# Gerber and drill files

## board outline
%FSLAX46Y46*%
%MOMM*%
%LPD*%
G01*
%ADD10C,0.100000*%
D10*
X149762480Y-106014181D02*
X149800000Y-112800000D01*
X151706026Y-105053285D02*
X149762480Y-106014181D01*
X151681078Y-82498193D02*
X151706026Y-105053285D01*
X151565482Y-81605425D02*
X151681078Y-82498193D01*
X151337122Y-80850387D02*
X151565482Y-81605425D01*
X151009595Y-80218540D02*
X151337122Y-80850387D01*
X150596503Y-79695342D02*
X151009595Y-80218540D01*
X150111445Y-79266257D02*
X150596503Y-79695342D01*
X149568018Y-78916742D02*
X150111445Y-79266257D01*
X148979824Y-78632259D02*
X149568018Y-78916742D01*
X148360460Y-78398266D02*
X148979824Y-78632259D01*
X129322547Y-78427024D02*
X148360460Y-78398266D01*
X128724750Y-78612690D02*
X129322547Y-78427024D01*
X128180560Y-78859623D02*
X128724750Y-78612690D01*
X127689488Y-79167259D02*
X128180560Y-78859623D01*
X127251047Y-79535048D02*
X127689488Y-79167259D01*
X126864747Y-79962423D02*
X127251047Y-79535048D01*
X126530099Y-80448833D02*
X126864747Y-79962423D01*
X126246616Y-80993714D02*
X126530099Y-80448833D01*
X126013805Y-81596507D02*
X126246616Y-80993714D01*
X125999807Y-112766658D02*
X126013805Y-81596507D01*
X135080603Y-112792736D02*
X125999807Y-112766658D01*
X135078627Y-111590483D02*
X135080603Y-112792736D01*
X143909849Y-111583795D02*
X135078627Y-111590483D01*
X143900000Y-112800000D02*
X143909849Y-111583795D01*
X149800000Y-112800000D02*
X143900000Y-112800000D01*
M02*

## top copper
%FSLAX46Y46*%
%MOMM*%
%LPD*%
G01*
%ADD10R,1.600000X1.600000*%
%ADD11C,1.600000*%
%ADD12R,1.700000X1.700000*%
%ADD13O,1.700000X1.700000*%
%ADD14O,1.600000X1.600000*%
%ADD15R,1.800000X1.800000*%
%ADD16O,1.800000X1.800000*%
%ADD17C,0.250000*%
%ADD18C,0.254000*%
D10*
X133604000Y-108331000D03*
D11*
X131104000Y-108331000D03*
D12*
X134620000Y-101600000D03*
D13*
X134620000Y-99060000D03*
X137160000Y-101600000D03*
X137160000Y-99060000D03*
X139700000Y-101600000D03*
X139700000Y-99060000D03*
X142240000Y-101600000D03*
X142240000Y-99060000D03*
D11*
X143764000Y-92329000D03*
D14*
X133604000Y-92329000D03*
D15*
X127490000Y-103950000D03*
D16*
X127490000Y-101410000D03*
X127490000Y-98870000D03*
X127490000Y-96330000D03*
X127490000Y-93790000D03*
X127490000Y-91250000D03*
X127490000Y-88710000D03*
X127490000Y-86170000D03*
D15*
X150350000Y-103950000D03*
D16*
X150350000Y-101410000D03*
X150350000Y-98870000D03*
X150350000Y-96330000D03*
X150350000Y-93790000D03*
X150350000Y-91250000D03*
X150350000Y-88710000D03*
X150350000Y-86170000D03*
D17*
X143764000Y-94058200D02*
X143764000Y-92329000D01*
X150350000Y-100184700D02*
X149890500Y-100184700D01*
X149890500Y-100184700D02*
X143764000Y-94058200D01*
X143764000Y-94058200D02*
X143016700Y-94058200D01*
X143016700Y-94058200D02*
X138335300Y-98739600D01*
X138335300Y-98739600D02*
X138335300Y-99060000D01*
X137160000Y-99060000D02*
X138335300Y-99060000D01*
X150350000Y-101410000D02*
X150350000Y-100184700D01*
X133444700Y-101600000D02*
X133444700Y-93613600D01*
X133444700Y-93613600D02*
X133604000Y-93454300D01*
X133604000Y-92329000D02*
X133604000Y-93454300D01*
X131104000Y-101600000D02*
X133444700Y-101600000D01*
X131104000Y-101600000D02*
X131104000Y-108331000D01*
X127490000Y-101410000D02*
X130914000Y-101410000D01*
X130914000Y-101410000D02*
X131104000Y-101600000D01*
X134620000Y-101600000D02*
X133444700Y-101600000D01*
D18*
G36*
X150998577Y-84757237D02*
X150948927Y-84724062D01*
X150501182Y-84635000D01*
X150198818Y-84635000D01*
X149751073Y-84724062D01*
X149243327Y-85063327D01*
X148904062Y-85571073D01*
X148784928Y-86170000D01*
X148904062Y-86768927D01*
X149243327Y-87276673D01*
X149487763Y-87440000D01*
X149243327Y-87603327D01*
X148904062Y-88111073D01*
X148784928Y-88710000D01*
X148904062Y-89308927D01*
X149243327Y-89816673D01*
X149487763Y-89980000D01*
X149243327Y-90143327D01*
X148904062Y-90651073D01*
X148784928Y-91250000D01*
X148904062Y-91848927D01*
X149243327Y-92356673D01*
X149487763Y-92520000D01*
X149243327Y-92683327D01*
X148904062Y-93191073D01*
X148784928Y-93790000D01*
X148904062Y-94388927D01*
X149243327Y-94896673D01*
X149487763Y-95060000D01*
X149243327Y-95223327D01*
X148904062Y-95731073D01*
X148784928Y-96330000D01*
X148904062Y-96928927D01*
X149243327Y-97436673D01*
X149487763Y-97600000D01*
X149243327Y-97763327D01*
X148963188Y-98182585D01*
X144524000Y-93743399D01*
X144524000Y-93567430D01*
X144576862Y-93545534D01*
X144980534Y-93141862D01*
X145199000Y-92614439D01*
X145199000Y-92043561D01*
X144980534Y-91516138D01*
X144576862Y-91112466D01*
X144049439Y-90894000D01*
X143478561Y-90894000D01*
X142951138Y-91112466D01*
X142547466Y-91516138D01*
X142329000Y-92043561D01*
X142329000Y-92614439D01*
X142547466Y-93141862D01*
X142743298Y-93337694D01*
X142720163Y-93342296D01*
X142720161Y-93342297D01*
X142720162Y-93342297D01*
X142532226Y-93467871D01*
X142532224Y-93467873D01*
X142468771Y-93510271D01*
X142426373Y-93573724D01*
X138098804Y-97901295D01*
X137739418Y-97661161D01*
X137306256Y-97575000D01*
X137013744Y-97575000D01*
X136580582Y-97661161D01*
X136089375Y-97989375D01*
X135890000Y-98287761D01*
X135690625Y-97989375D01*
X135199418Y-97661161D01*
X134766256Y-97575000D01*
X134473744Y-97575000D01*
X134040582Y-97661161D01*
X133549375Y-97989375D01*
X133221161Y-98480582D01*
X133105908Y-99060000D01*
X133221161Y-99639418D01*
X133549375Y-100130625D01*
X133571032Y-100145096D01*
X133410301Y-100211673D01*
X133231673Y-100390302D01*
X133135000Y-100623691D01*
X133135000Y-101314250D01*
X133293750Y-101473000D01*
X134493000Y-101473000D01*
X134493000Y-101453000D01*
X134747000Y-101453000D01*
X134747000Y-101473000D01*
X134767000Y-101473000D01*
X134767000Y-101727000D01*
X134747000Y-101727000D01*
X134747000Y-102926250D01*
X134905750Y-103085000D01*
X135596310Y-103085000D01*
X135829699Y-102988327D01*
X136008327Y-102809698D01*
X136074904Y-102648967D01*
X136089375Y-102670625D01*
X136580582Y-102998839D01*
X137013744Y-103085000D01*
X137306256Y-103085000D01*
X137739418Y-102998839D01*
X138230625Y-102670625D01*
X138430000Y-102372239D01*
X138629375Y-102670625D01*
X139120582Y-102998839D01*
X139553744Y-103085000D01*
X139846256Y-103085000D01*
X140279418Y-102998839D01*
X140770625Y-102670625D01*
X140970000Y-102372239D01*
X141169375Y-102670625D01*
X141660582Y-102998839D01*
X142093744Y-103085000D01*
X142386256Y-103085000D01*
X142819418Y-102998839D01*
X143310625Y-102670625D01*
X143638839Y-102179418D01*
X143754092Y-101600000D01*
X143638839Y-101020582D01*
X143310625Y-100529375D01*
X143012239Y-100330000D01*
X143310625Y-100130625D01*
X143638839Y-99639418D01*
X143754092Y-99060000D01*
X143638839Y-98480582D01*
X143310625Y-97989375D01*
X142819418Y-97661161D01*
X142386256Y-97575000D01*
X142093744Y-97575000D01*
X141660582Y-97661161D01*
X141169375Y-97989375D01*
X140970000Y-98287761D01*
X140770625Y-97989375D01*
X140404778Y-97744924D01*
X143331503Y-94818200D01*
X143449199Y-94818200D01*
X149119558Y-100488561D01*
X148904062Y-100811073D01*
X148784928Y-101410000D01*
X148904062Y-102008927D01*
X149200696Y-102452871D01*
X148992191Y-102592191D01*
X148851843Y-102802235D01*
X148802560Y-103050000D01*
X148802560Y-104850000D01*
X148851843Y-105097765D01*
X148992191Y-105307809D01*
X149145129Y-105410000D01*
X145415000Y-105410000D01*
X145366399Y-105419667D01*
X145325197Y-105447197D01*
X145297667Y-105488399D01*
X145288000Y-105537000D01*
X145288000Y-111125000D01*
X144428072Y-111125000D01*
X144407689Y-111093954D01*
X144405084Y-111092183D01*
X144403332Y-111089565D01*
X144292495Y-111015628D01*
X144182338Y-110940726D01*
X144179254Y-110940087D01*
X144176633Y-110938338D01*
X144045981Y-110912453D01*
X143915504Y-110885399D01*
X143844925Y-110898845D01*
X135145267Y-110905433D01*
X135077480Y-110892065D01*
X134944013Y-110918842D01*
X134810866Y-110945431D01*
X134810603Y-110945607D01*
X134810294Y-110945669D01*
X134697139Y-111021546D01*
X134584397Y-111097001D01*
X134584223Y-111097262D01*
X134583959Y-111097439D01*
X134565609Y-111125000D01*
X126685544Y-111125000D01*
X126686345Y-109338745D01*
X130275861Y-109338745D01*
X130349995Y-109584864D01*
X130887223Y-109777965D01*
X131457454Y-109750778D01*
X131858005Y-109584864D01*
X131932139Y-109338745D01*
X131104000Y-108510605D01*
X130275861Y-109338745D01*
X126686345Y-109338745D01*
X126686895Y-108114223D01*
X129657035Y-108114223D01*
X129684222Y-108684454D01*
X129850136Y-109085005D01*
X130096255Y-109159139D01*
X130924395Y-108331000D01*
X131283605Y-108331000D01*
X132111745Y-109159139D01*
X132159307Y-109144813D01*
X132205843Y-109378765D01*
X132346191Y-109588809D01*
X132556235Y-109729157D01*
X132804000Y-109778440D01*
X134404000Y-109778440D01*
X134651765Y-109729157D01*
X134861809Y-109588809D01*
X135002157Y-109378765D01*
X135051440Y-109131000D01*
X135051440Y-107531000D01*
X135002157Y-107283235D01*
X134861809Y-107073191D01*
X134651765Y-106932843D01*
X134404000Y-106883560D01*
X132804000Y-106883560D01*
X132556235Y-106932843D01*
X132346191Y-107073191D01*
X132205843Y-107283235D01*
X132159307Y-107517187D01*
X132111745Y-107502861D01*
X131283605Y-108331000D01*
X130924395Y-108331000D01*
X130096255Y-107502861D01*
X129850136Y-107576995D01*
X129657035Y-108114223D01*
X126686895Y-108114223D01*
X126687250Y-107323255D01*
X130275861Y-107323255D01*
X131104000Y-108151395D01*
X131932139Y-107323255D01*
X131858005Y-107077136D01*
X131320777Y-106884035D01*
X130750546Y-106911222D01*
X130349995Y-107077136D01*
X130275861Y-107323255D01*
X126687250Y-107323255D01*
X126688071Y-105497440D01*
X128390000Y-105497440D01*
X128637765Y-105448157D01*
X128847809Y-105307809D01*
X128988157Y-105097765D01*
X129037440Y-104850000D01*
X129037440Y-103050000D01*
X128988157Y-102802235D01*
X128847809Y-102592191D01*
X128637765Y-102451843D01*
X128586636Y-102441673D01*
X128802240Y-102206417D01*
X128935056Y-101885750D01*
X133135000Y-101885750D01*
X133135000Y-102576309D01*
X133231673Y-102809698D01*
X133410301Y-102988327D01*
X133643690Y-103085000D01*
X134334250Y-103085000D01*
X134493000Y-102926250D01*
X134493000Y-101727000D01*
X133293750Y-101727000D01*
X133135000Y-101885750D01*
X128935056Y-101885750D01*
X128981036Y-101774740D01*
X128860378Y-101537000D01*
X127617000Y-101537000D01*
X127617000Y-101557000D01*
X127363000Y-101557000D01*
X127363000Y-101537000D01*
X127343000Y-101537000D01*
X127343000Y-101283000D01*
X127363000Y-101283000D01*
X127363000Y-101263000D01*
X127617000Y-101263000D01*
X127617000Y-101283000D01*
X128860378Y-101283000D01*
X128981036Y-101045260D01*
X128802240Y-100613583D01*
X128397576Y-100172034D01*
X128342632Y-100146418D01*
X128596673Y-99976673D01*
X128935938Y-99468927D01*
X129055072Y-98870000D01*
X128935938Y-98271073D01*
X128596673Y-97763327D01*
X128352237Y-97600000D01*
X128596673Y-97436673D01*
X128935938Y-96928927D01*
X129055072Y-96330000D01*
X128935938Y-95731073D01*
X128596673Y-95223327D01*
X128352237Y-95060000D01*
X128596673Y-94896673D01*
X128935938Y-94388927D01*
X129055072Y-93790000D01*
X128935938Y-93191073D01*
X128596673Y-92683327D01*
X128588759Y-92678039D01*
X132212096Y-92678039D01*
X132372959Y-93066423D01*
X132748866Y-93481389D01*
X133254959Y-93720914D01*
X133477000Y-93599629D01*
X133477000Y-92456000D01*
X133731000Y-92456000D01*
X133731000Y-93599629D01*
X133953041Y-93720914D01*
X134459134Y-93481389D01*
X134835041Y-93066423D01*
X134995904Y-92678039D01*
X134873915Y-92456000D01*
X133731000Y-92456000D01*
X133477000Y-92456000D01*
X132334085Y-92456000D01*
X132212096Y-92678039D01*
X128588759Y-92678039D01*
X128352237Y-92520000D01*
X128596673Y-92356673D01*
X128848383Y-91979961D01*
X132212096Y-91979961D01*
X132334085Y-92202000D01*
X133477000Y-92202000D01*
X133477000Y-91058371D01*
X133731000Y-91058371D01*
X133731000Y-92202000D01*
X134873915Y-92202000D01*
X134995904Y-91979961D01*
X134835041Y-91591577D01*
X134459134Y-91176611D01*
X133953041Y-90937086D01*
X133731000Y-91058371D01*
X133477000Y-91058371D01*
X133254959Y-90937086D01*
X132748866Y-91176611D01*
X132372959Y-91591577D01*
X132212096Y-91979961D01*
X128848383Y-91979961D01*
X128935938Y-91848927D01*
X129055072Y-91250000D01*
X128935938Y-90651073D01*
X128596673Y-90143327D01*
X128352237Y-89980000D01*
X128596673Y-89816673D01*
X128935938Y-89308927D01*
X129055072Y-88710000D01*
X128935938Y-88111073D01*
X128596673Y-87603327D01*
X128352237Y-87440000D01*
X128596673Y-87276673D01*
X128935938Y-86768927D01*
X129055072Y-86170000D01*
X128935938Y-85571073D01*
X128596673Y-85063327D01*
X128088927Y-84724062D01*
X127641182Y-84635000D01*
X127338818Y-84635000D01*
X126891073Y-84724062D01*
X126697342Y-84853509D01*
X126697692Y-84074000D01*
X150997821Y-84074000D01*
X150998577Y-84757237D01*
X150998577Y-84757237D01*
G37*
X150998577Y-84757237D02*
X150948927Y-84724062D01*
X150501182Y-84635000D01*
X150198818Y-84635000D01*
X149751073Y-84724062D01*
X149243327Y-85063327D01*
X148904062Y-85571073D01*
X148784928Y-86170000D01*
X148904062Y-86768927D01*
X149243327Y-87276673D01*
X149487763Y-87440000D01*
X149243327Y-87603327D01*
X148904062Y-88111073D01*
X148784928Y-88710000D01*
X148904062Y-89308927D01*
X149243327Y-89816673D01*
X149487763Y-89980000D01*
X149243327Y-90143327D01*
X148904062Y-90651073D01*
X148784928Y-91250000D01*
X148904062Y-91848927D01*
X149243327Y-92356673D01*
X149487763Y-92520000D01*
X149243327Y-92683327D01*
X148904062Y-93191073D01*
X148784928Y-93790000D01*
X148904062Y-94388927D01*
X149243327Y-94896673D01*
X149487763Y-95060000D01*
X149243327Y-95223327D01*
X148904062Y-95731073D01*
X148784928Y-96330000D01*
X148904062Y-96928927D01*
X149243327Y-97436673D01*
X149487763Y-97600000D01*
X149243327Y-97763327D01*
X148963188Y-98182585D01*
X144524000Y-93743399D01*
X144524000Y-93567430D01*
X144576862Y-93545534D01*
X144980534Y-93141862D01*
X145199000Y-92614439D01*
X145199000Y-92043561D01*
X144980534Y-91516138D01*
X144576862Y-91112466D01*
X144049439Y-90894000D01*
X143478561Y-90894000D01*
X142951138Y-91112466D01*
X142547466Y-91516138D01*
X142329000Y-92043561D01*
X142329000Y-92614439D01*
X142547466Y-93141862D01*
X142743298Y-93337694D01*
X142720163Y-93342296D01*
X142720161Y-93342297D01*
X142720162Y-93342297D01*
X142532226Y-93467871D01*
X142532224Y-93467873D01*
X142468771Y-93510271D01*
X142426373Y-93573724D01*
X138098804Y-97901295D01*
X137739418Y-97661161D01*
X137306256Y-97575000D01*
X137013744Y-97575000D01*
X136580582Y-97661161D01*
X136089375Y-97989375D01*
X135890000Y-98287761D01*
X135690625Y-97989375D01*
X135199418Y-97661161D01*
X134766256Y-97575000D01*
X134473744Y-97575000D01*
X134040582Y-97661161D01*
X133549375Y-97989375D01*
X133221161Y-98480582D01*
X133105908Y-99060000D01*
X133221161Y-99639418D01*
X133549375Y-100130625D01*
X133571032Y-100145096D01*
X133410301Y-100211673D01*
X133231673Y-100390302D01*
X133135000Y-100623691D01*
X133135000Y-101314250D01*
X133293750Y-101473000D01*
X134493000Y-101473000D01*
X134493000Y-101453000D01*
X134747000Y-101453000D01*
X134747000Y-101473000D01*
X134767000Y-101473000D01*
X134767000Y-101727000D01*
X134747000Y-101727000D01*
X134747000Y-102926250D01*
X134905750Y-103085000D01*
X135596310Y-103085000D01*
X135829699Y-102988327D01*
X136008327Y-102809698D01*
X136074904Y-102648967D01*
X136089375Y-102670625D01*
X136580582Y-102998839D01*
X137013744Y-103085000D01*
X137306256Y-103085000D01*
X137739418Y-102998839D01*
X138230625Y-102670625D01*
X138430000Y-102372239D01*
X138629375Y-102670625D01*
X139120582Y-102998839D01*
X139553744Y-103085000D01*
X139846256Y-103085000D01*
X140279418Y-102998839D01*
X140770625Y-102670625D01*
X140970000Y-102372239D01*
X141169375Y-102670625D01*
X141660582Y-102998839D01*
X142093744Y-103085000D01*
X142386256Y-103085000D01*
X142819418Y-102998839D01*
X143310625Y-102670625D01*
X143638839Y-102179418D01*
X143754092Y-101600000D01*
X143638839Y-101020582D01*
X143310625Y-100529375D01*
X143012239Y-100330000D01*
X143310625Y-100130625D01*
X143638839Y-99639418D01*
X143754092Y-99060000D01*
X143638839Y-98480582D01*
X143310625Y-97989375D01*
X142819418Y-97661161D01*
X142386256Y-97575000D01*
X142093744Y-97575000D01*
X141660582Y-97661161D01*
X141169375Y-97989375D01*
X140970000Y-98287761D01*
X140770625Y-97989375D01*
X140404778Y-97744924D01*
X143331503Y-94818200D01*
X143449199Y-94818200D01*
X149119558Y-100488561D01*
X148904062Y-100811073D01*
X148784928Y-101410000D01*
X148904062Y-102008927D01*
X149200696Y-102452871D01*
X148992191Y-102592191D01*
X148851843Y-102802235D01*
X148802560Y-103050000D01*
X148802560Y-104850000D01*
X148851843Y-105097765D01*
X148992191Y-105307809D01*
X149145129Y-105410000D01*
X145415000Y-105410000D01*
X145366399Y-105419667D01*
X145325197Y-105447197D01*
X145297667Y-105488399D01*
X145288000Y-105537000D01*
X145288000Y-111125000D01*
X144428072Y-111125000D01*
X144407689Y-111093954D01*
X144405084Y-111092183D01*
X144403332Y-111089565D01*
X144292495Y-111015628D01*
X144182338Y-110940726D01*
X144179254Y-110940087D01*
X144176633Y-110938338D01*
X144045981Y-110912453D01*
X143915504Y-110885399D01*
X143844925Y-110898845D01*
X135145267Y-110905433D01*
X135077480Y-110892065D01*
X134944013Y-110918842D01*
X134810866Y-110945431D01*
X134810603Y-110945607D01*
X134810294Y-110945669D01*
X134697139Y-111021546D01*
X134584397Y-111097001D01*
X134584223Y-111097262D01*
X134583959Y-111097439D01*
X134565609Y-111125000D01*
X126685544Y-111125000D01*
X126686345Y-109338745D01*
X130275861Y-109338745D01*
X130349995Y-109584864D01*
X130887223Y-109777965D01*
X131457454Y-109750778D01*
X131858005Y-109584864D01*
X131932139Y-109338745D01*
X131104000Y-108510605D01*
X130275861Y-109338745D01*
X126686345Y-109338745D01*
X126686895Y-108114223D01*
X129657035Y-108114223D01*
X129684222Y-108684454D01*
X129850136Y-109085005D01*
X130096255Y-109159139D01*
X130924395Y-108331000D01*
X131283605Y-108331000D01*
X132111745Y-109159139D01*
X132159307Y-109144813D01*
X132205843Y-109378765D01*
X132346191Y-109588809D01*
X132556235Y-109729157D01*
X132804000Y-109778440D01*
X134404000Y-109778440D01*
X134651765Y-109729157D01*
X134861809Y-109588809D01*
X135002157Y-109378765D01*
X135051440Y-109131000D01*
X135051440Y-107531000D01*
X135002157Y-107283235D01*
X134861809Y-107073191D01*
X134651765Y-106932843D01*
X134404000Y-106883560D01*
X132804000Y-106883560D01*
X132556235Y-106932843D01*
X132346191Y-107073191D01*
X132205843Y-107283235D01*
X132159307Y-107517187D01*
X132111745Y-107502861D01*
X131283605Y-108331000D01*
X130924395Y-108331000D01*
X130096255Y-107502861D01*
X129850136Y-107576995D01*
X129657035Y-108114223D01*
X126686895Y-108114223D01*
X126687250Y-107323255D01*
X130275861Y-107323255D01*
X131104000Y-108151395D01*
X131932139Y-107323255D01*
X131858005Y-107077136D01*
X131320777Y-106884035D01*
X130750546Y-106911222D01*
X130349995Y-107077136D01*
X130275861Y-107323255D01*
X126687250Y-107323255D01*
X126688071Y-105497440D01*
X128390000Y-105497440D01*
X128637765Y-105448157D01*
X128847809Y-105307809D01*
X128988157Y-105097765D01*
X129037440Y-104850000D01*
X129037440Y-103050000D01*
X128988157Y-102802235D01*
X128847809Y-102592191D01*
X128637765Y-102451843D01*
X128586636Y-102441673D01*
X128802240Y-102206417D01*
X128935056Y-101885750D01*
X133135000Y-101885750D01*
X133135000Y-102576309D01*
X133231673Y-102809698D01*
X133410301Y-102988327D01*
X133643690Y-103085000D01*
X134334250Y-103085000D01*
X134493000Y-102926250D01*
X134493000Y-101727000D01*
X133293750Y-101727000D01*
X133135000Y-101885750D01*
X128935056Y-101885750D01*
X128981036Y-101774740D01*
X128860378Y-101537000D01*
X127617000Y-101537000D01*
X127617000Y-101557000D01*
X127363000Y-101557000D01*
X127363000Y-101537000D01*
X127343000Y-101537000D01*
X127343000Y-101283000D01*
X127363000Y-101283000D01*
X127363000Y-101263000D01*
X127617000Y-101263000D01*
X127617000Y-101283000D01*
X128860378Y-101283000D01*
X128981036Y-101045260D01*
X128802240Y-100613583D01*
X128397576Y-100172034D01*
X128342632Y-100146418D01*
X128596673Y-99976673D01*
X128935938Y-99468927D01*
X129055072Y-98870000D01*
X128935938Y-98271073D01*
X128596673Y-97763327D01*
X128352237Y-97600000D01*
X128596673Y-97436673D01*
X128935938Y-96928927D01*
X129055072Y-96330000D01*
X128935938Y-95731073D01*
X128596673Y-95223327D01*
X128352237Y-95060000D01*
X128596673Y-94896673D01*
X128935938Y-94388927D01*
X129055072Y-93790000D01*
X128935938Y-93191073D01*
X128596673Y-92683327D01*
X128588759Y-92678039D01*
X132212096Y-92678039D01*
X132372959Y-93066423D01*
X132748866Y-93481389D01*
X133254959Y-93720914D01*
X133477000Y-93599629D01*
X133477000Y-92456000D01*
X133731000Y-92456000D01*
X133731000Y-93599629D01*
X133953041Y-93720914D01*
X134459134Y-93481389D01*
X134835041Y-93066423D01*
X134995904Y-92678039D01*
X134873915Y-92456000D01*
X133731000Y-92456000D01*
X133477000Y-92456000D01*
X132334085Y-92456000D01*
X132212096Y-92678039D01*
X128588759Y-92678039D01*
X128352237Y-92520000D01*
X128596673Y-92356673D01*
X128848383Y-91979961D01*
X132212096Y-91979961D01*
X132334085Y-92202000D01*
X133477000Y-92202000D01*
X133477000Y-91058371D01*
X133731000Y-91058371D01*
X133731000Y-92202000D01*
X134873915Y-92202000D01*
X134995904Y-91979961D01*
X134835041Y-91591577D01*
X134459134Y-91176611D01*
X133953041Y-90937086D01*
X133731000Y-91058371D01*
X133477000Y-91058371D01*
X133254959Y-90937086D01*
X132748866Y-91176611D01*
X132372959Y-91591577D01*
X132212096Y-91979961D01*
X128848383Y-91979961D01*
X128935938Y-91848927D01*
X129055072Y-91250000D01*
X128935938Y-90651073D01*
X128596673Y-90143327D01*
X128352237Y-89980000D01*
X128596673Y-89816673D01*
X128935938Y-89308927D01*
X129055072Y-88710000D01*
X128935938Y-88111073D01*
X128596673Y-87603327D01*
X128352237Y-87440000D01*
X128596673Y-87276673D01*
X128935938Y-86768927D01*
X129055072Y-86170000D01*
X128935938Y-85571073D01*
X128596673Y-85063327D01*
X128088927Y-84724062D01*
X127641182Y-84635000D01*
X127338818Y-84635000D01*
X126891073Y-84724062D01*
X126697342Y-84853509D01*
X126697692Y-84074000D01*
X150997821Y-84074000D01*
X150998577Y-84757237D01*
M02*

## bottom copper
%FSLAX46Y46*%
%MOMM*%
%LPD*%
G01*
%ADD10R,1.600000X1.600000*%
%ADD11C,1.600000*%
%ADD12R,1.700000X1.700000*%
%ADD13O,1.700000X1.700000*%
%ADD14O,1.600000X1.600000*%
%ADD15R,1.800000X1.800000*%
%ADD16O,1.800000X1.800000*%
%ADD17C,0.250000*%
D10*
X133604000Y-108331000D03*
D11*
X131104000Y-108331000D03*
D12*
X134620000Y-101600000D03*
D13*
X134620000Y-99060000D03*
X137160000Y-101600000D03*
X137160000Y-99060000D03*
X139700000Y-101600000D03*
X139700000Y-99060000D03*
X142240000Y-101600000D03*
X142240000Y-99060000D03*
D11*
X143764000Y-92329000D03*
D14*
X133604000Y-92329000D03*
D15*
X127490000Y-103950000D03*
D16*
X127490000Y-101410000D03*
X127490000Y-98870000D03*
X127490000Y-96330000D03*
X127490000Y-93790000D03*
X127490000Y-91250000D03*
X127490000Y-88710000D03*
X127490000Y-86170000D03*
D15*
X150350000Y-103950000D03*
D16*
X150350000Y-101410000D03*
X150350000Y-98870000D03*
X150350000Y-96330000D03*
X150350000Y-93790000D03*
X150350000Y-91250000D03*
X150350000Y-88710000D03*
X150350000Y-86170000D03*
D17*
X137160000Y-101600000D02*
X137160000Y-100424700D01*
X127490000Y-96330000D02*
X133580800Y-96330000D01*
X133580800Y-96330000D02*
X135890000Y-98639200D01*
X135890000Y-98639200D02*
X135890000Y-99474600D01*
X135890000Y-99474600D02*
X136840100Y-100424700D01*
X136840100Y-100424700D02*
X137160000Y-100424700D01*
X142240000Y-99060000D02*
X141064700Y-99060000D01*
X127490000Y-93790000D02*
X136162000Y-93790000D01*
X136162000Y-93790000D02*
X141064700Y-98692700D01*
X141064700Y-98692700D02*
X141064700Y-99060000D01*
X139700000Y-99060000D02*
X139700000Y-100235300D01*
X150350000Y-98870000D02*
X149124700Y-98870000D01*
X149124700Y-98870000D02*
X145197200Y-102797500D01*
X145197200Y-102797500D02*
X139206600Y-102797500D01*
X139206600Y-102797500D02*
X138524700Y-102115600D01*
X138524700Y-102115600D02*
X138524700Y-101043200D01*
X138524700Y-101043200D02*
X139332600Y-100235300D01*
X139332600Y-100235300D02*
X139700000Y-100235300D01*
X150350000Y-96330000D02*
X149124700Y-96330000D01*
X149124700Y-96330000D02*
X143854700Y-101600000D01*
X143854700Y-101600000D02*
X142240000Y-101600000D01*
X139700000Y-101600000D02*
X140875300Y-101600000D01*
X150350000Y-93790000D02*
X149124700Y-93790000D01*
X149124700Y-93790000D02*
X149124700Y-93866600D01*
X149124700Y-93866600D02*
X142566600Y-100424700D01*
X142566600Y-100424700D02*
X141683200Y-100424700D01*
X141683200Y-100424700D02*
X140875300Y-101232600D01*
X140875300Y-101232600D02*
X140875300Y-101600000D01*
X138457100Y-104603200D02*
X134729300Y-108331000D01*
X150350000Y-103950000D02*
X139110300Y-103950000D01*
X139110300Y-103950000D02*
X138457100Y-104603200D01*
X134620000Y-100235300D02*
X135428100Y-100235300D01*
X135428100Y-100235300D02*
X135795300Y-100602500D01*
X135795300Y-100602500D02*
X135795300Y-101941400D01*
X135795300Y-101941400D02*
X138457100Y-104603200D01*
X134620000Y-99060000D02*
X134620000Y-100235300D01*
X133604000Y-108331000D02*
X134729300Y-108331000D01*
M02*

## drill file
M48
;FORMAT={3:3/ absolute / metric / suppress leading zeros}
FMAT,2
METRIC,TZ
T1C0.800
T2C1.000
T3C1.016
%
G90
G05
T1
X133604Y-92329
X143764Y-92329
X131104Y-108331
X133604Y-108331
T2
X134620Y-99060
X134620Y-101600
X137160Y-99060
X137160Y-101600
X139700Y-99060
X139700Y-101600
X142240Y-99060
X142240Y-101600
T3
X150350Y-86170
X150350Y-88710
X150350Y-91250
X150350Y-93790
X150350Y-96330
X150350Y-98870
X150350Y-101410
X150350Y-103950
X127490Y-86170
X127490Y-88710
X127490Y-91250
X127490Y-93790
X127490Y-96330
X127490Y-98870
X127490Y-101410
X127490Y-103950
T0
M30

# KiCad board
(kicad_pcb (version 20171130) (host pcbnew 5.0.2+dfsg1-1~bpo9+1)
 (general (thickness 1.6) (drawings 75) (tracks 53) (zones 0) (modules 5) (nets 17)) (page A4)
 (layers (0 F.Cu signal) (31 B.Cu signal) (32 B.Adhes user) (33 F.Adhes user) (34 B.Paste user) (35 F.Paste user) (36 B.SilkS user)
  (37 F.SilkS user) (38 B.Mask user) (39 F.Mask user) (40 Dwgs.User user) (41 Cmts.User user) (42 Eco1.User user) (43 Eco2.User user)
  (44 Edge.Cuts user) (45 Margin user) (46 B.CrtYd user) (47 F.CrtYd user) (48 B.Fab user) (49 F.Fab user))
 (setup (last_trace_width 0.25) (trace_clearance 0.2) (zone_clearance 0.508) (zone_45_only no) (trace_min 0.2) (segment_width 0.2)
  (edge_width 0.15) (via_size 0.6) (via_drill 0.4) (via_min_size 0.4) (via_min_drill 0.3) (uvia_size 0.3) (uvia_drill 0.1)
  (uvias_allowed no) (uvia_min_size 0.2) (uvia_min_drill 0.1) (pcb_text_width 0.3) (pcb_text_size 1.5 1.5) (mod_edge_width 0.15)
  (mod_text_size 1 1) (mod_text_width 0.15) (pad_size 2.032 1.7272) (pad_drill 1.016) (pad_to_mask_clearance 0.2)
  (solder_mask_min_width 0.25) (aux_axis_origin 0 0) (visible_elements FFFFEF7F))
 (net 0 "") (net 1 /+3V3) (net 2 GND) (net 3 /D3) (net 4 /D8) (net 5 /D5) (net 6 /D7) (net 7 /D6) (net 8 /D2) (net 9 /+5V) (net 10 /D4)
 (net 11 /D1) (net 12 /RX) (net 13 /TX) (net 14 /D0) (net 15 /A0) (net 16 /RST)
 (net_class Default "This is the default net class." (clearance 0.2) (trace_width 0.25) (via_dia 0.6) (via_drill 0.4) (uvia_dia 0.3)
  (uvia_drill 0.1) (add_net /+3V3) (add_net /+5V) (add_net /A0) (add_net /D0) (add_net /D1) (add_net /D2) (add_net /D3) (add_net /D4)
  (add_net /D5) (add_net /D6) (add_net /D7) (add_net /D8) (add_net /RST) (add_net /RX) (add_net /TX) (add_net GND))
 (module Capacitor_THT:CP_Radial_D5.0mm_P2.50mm (layer F.Cu) (at 133.604 108.331 180)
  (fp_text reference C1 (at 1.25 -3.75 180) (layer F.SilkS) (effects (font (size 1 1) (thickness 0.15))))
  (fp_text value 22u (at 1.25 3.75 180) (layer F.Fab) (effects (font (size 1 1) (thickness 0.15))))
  (pad 1 thru_hole rect (at 0 0 180) (size 1.6 1.6) (drill 0.8) (layers *.Cu *.Mask) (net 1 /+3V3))
  (pad 2 thru_hole circle (at 2.5 0 180) (size 1.6 1.6) (drill 0.8) (layers *.Cu *.Mask) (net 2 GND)))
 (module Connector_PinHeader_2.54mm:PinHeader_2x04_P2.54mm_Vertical (layer F.Cu) (at 134.62 101.6 90)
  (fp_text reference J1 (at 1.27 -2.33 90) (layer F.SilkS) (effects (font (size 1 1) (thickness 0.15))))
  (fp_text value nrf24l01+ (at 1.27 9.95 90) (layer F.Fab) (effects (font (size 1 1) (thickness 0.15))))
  (pad 1 thru_hole rect (at 0 0 90) (size 1.7 1.7) (drill 1) (layers *.Cu *.Mask) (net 2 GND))
  (pad 2 thru_hole oval (at 2.54 0 90) (size 1.7 1.7) (drill 1) (layers *.Cu *.Mask) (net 1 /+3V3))
  (pad 3 thru_hole oval (at 0 2.54 90) (size 1.7 1.7) (drill 1) (layers *.Cu *.Mask) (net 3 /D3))
  (pad 4 thru_hole oval (at 2.54 2.54 90) (size 1.7 1.7) (drill 1) (layers *.Cu *.Mask) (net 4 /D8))
  (pad 5 thru_hole oval (at 0 5.08 90) (size 1.7 1.7) (drill 1) (layers *.Cu *.Mask) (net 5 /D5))
  (pad 6 thru_hole oval (at 2.54 5.08 90) (size 1.7 1.7) (drill 1) (layers *.Cu *.Mask) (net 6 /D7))
  (pad 7 thru_hole oval (at 0 7.62 90) (size 1.7 1.7) (drill 1) (layers *.Cu *.Mask) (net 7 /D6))
  (pad 8 thru_hole oval (at 2.54 7.62 90) (size 1.7 1.7) (drill 1) (layers *.Cu *.Mask) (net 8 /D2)))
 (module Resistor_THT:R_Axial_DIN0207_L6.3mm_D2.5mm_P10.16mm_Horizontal (layer F.Cu) (at 143.764 92.329 180)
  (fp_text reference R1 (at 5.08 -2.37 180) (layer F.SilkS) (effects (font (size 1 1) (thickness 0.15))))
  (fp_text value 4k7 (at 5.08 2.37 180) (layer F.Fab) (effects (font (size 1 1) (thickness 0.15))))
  (pad 1 thru_hole circle (at 0 0 180) (size 1.6 1.6) (drill 0.8) (layers *.Cu *.Mask) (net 4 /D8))
  (pad 2 thru_hole oval (at 10.16 0 180) (size 1.6 1.6) (drill 0.8) (layers *.Cu *.Mask) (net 2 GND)))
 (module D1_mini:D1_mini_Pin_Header (layer F.Cu) (at 127.49 103.95 180)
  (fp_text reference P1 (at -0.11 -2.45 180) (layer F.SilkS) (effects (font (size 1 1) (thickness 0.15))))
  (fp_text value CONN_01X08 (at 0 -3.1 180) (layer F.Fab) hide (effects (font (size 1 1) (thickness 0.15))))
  (pad 1 thru_hole rect (at 0 0 180) (size 1.8 1.8) (drill 1.016) (layers *.Cu *.Mask F.SilkS) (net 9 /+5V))
  (pad 2 thru_hole oval (at 0 2.54 180) (size 1.8 1.8) (drill 1.016) (layers *.Cu *.Mask F.SilkS) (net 2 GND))
  (pad 3 thru_hole oval (at 0 5.08 180) (size 1.8 1.8) (drill 1.016) (layers *.Cu *.Mask F.SilkS) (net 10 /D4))
  (pad 4 thru_hole oval (at 0 7.62 180) (size 1.8 1.8) (drill 1.016) (layers *.Cu *.Mask F.SilkS) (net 3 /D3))
  (pad 5 thru_hole oval (at 0 10.16 180) (size 1.8 1.8) (drill 1.016) (layers *.Cu *.Mask F.SilkS) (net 8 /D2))
  (pad 6 thru_hole oval (at 0 12.7 180) (size 1.8 1.8) (drill 1.016) (layers *.Cu *.Mask F.SilkS) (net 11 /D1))
  (pad 7 thru_hole oval (at 0 15.24 180) (size 1.8 1.8) (drill 1.016) (layers *.Cu *.Mask F.SilkS) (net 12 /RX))
  (pad 8 thru_hole oval (at 0 17.78 180) (size 1.8 1.8) (drill 1.016) (layers *.Cu *.Mask F.SilkS) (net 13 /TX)))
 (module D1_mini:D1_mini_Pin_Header (layer F.Cu) (at 150.35 103.95 180)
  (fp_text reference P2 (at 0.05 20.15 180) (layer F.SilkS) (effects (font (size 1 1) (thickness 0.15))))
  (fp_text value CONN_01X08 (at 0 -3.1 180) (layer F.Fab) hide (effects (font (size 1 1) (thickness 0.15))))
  (pad 1 thru_hole rect (at 0 0 180) (size 1.8 1.8) (drill 1.016) (layers *.Cu *.Mask F.SilkS) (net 1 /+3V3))
  (pad 2 thru_hole oval (at 0 2.54 180) (size 1.8 1.8) (drill 1.016) (layers *.Cu *.Mask F.SilkS) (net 4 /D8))
  (pad 3 thru_hole oval (at 0 5.08 180) (size 1.8 1.8) (drill 1.016) (layers *.Cu *.Mask F.SilkS) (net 6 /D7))
  (pad 4 thru_hole oval (at 0 7.62 180) (size 1.8 1.8) (drill 1.016) (layers *.Cu *.Mask F.SilkS) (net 7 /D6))
  (pad 5 thru_hole oval (at 0 10.16 180) (size 1.8 1.8) (drill 1.016) (layers *.Cu *.Mask F.SilkS) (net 5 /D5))
  (pad 6 thru_hole oval (at 0 12.7 180) (size 1.8 1.8) (drill 1.016) (layers *.Cu *.Mask F.SilkS) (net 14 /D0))
  (pad 7 thru_hole oval (at 0 15.24 180) (size 1.8 1.8) (drill 1.016) (layers *.Cu *.Mask F.SilkS) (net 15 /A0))
  (pad 8 thru_hole oval (at 0 17.78 180) (size 1.8 1.8) (drill 1.016) (layers *.Cu *.Mask F.SilkS) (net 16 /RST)))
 (gr_line (start 149.76248 106.014181) (end 149.8 112.8) (layer Edge.Cuts) (width 0.1))
 (gr_line (start 151.706026 105.053285) (end 149.76248 106.014181) (layer Edge.Cuts) (width 0.1))
 (gr_line (start 151.681078 82.498193) (end 151.706026 105.053285) (layer Edge.Cuts) (width 0.1))
 (gr_line (start 151.565482 81.605425) (end 151.681078 82.498193) (layer Edge.Cuts) (width 0.1))
 (gr_line (start 151.337122 80.850387) (end 151.565482 81.605425) (layer Edge.Cuts) (width 0.1))
 (gr_line (start 151.009595 80.21854) (end 151.337122 80.850387) (layer Edge.Cuts) (width 0.1))
 (gr_line (start 150.596503 79.695342) (end 151.009595 80.21854) (layer Edge.Cuts) (width 0.1))
 (gr_line (start 150.111445 79.266257) (end 150.596503 79.695342) (layer Edge.Cuts) (width 0.1))
 (gr_line (start 149.568018 78.916742) (end 150.111445 79.266257) (layer Edge.Cuts) (width 0.1))
 (gr_line (start 148.979824 78.632259) (end 149.568018 78.916742) (layer Edge.Cuts) (width 0.1))
 (gr_line (start 148.36046 78.398266) (end 148.979824 78.632259) (layer Edge.Cuts) (width 0.1))
 (gr_line (start 129.322547 78.427024) (end 148.36046 78.398266) (layer Edge.Cuts) (width 0.1))
 (gr_line (start 128.72475 78.61269) (end 129.322547 78.427024) (layer Edge.Cuts) (width 0.1))
 (gr_line (start 128.18056 78.859623) (end 128.72475 78.61269) (layer Edge.Cuts) (width 0.1))
 (gr_line (start 127.689488 79.167259) (end 128.18056 78.859623) (layer Edge.Cuts) (width 0.1))
 (gr_line (start 127.251047 79.535048) (end 127.689488 79.167259) (layer Edge.Cuts) (width 0.1))
 (gr_line (start 126.864747 79.962423) (end 127.251047 79.535048) (layer Edge.Cuts) (width 0.1))
 (gr_line (start 126.530099 80.448833) (end 126.864747 79.962423) (layer Edge.Cuts) (width 0.1))
 (gr_line (start 126.246616 80.993714) (end 126.530099 80.448833) (layer Edge.Cuts) (width 0.1))
 (gr_line (start 126.013805 81.596507) (end 126.246616 80.993714) (layer Edge.Cuts) (width 0.1))
 (gr_line (start 125.999807 112.766658) (end 126.013805 81.596507) (layer Edge.Cuts) (width 0.1))
 (gr_line (start 135.080603 112.792736) (end 125.999807 112.766658) (layer Edge.Cuts) (width 0.1))
 (gr_line (start 135.078627 111.590483) (end 135.080603 112.792736) (layer Edge.Cuts) (width 0.1))
 (gr_line (start 143.909849 111.583795) (end 135.078627 111.590483) (layer Edge.Cuts) (width 0.1))
 (gr_line (start 143.9 112.8) (end 143.909849 111.583795) (layer Edge.Cuts) (width 0.1))
 (gr_line (start 149.8 112.8) (end 143.9 112.8) (layer Edge.Cuts) (width 0.1))
 (segment (start 137.16 101.6) (end 137.16 100.4247) (width 0.25) (layer B.Cu) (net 3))
 (segment (start 127.49 96.33) (end 133.5808 96.33) (width 0.25) (layer B.Cu) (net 3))
 (segment (start 133.5808 96.33) (end 135.89 98.6392) (width 0.25) (layer B.Cu) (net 3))
 (segment (start 135.89 98.6392) (end 135.89 99.4746) (width 0.25) (layer B.Cu) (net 3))
 (segment (start 135.89 99.4746) (end 136.8401 100.4247) (width 0.25) (layer B.Cu) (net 3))
 (segment (start 136.8401 100.4247) (end 137.16 100.4247) (width 0.25) (layer B.Cu) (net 3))
 (segment (start 142.24 99.06) (end 141.0647 99.06) (width 0.25) (layer B.Cu) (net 8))
 (segment (start 127.49 93.79) (end 136.162 93.79) (width 0.25) (layer B.Cu) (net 8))
 (segment (start 136.162 93.79) (end 141.0647 98.6927) (width 0.25) (layer B.Cu) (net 8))
 (segment (start 141.0647 98.6927) (end 141.0647 99.06) (width 0.25) (layer B.Cu) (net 8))
 (segment (start 143.764 94.0582) (end 143.764 92.329) (width 0.25) (layer F.Cu) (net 4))
 (segment (start 150.35 100.1847) (end 149.8905 100.1847) (width 0.25) (layer F.Cu) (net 4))
 (segment (start 149.8905 100.1847) (end 143.764 94.0582) (width 0.25) (layer F.Cu) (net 4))
 (segment (start 143.764 94.0582) (end 143.0167 94.0582) (width 0.25) (layer F.Cu) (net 4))
 (segment (start 143.0167 94.0582) (end 138.3353 98.7396) (width 0.25) (layer F.Cu) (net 4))
 (segment (start 138.3353 98.7396) (end 138.3353 99.06) (width 0.25) (layer F.Cu) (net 4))
 (segment (start 137.16 99.06) (end 138.3353 99.06) (width 0.25) (layer F.Cu) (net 4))
 (segment (start 150.35 101.41) (end 150.35 100.1847) (width 0.25) (layer F.Cu) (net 4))
 (segment (start 139.7 99.06) (end 139.7 100.2353) (width 0.25) (layer B.Cu) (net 6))
 (segment (start 150.35 98.87) (end 149.1247 98.87) (width 0.25) (layer B.Cu) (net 6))
 (segment (start 149.1247 98.87) (end 145.1972 102.7975) (width 0.25) (layer B.Cu) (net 6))
 (segment (start 145.1972 102.7975) (end 139.2066 102.7975) (width 0.25) (layer B.Cu) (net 6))
 (segment (start 139.2066 102.7975) (end 138.5247 102.1156) (width 0.25) (layer B.Cu) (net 6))
 (segment (start 138.5247 102.1156) (end 138.5247 101.0432) (width 0.25) (layer B.Cu) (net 6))
 (segment (start 138.5247 101.0432) (end 139.3326 100.2353) (width 0.25) (layer B.Cu) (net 6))
 (segment (start 139.3326 100.2353) (end 139.7 100.2353) (width 0.25) (layer B.Cu) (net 6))
 (segment (start 150.35 96.33) (end 149.1247 96.33) (width 0.25) (layer B.Cu) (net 7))
 (segment (start 149.1247 96.33) (end 143.8547 101.6) (width 0.25) (layer B.Cu) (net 7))
 (segment (start 143.8547 101.6) (end 142.24 101.6) (width 0.25) (layer B.Cu) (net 7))
 (segment (start 139.7 101.6) (end 140.8753 101.6) (width 0.25) (layer B.Cu) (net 5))
 (segment (start 150.35 93.79) (end 149.1247 93.79) (width 0.25) (layer B.Cu) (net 5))
 (segment (start 149.1247 93.79) (end 149.1247 93.8666) (width 0.25) (layer B.Cu) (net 5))
 (segment (start 149.1247 93.8666) (end 142.5666 100.4247) (width 0.25) (layer B.Cu) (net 5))
 (segment (start 142.5666 100.4247) (end 141.6832 100.4247) (width 0.25) (layer B.Cu) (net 5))
 (segment (start 141.6832 100.4247) (end 140.8753 101.2326) (width 0.25) (layer B.Cu) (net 5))
 (segment (start 140.8753 101.2326) (end 140.8753 101.6) (width 0.25) (layer B.Cu) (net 5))
 (segment (start 133.4447 101.6) (end 133.4447 93.6136) (width 0.25) (layer F.Cu) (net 2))
 (segment (start 133.4447 93.6136) (end 133.604 93.4543) (width 0.25) (layer F.Cu) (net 2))
 (segment (start 133.604 92.329) (end 133.604 93.4543) (width 0.25) (layer F.Cu) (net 2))
 (segment (start 131.104 101.6) (end 133.4447 101.6) (width 0.25) (layer F.Cu) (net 2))
 (segment (start 131.104 101.6) (end 131.104 108.331) (width 0.25) (layer F.Cu) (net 2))
 (segment (start 127.49 101.41) (end 130.914 101.41) (width 0.25) (layer F.Cu) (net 2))
 (segment (start 130.914 101.41) (end 131.104 101.6) (width 0.25) (layer F.Cu) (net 2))
 (segment (start 134.62 101.6) (end 133.4447 101.6) (width 0.25) (layer F.Cu) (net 2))
 (segment (start 138.4571 104.6032) (end 134.7293 108.331) (width 0.25) (layer B.Cu) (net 1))
 (segment (start 150.35 103.95) (end 139.1103 103.95) (width 0.25) (layer B.Cu) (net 1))
 (segment (start 139.1103 103.95) (end 138.4571 104.6032) (width 0.25) (layer B.Cu) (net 1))
 (segment (start 134.62 100.2353) (end 135.4281 100.2353) (width 0.25) (layer B.Cu) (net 1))
 (segment (start 135.4281 100.2353) (end 135.7953 100.6025) (width 0.25) (layer B.Cu) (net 1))
 (segment (start 135.7953 100.6025) (end 135.7953 101.9414) (width 0.25) (layer B.Cu) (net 1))
 (segment (start 135.7953 101.9414) (end 138.4571 104.6032) (width 0.25) (layer B.Cu) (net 1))
 (segment (start 134.62 99.06) (end 134.62 100.2353) (width 0.25) (layer B.Cu) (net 1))
 (segment (start 133.604 108.331) (end 134.7293 108.331) (width 0.25) (layer B.Cu) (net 1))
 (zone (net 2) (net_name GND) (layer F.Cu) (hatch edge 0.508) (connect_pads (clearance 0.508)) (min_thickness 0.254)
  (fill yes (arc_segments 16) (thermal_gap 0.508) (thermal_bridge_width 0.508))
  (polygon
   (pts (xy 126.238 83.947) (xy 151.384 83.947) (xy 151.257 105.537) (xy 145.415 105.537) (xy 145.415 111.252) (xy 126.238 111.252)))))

